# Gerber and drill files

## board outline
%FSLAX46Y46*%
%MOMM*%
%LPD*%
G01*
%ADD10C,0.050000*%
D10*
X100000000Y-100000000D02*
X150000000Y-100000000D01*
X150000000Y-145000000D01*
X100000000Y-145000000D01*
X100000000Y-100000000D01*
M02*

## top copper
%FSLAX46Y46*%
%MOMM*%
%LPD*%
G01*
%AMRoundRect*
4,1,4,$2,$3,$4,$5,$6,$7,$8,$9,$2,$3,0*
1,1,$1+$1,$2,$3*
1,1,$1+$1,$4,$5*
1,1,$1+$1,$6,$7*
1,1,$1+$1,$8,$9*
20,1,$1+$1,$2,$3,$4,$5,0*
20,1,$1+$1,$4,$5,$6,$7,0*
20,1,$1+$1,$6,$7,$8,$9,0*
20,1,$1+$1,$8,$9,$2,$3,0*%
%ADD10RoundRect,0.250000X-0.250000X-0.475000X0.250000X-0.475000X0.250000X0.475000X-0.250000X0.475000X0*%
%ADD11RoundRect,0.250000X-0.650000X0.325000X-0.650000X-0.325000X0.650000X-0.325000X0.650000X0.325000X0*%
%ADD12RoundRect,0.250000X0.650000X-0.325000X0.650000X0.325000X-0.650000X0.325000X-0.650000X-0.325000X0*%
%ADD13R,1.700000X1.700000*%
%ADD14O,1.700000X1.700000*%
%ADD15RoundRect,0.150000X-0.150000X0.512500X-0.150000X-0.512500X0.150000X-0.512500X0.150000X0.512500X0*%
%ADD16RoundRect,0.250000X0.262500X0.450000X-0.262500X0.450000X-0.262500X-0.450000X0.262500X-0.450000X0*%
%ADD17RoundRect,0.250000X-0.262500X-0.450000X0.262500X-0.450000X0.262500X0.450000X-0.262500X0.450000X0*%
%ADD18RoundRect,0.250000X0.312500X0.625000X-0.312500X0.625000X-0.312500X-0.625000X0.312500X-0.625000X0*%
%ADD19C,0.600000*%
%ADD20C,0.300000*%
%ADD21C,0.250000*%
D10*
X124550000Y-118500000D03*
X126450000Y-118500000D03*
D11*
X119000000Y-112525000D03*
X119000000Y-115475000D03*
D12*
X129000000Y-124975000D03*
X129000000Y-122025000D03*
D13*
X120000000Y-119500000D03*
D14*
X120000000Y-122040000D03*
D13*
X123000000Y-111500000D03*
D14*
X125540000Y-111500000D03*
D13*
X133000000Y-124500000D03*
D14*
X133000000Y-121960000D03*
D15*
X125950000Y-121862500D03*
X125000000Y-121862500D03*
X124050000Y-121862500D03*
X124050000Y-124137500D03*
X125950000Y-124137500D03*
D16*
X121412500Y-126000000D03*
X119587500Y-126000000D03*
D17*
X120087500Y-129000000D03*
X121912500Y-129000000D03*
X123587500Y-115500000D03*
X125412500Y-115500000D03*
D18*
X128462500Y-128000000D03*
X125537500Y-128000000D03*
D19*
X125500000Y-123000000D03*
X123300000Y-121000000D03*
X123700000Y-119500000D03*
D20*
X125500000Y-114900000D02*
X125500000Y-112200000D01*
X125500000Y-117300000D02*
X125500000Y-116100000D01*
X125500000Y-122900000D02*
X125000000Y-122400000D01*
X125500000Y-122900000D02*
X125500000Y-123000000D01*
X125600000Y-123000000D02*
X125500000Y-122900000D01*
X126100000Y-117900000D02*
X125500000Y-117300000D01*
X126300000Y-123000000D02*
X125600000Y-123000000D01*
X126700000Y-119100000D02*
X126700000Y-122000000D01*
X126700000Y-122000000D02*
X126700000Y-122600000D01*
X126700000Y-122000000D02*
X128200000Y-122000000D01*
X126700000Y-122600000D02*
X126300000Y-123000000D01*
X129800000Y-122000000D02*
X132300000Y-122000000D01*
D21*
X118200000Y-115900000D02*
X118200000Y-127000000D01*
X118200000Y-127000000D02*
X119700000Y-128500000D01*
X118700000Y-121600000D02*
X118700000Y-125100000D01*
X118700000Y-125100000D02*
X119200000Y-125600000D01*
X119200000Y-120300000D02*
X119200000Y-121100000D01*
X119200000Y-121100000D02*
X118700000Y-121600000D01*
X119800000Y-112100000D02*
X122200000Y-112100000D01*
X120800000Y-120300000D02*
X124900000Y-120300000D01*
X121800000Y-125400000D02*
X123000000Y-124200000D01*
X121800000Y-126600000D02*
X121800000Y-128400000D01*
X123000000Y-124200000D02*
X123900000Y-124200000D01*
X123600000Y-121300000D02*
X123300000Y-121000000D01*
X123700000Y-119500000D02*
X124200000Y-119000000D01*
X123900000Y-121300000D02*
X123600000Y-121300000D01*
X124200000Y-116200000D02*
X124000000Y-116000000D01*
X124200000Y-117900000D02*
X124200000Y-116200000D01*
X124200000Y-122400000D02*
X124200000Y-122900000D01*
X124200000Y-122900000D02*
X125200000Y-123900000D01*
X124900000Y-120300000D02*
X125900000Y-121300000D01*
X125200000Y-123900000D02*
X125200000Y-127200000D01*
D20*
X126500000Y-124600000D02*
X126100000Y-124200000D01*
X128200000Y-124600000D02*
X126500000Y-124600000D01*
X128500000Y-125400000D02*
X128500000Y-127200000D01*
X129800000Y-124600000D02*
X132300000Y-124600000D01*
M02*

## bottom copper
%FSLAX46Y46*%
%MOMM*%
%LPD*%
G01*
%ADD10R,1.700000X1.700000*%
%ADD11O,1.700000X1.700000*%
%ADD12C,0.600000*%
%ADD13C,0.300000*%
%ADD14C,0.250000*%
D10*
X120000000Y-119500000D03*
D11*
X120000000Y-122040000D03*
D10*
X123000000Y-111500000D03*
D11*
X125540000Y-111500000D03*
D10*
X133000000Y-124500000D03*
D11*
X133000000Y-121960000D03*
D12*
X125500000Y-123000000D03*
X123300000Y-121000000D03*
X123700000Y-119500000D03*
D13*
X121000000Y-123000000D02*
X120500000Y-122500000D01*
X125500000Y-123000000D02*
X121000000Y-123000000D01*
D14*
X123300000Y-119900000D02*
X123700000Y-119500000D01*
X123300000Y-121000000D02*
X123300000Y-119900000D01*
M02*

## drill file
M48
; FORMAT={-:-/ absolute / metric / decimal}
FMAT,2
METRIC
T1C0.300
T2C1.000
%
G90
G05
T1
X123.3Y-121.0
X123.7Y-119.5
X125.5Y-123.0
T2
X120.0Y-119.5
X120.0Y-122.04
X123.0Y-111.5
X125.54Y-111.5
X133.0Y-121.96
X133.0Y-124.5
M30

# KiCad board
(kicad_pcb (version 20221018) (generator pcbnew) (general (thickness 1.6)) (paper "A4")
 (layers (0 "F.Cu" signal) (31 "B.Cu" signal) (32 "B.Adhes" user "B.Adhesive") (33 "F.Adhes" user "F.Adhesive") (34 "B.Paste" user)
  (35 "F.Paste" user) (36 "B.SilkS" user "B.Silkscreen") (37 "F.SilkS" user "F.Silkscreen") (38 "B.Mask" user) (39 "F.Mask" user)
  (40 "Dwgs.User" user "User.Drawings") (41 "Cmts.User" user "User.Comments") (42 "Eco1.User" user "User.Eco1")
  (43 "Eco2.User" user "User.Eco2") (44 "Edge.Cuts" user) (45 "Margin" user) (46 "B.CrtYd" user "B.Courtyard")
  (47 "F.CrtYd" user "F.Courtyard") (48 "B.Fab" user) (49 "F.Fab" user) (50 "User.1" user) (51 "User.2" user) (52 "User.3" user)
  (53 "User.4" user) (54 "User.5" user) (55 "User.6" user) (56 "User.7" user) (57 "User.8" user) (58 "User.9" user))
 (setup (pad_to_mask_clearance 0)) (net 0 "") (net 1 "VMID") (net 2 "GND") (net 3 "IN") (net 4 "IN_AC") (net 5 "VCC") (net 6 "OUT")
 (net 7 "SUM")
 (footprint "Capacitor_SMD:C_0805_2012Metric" (layer "F.Cu") (at 125.5 118.5)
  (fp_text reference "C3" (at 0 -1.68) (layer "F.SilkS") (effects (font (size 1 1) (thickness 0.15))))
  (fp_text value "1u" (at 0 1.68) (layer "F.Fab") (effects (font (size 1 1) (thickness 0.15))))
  (pad "1" smd roundrect (at -0.95 0) (size 1 1.45) (layers "F.Cu" "F.Paste" "F.Mask") (roundrect_rratio 0.25) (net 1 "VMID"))
  (pad "2" smd roundrect (at 0.95 0) (size 1 1.45) (layers "F.Cu" "F.Paste" "F.Mask") (roundrect_rratio 0.25) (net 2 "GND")))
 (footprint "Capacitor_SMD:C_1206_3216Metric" (layer "F.Cu") (at 119 114 -90)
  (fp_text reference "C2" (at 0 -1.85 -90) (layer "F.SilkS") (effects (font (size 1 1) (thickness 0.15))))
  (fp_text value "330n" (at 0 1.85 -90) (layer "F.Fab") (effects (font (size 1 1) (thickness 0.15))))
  (pad "1" smd roundrect (at -1.475 0 270) (size 1.15 1.8) (layers "F.Cu" "F.Paste" "F.Mask") (roundrect_rratio 0.217391) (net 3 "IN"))
  (pad "2" smd roundrect (at 1.475 0 270) (size 1.15 1.8) (layers "F.Cu" "F.Paste" "F.Mask") (roundrect_rratio 0.217391) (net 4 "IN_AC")))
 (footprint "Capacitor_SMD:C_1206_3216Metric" (layer "F.Cu") (at 129 123.5 90)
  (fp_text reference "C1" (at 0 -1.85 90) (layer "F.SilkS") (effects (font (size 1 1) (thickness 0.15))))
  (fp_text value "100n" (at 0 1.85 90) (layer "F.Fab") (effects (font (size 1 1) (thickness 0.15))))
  (pad "1" smd roundrect (at -1.475 0 90) (size 1.15 1.8) (layers "F.Cu" "F.Paste" "F.Mask") (roundrect_rratio 0.217391) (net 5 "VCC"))
  (pad "2" smd roundrect (at 1.475 0 90) (size 1.15 1.8) (layers "F.Cu" "F.Paste" "F.Mask") (roundrect_rratio 0.217391) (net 2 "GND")))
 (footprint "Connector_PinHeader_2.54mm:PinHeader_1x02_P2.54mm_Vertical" (layer "F.Cu") (at 120 119.5)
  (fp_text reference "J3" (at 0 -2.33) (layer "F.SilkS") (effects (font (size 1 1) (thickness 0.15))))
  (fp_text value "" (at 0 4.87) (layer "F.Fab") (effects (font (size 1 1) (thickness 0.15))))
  (pad "1" thru_hole rect (at 0 0) (size 1.7 1.7) (drill 1) (layers "*.Cu" "*.Mask") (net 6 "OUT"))
  (pad "2" thru_hole oval (at 0 2.54) (size 1.7 1.7) (drill 1) (layers "*.Cu" "*.Mask") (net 2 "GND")))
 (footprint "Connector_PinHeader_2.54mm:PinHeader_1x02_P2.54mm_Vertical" (layer "F.Cu") (at 123 111.5 90)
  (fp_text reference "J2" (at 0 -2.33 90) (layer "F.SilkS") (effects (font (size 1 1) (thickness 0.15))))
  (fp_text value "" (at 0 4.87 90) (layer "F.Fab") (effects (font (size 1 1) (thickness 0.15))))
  (pad "1" thru_hole rect (at 0 0 90) (size 1.7 1.7) (drill 1) (layers "*.Cu" "*.Mask") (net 3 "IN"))
  (pad "2" thru_hole oval (at 0 2.54 90) (size 1.7 1.7) (drill 1) (layers "*.Cu" "*.Mask") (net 2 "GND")))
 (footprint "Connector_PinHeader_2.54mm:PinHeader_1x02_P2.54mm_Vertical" (layer "F.Cu") (at 133 124.5 180)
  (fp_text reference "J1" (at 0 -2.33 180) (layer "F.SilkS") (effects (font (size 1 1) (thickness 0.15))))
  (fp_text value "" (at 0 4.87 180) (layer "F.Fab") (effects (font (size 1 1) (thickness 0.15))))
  (pad "1" thru_hole rect (at 0 0 180) (size 1.7 1.7) (drill 1) (layers "*.Cu" "*.Mask") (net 5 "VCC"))
  (pad "2" thru_hole oval (at 0 2.54 180) (size 1.7 1.7) (drill 1) (layers "*.Cu" "*.Mask") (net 2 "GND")))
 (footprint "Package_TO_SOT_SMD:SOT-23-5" (layer "F.Cu") (at 125 123 -90)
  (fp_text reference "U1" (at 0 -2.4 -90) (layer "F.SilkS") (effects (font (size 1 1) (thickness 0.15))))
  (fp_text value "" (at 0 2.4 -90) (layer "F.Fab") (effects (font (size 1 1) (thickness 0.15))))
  (pad "1" smd roundrect (at -1.1375 -0.95 270) (size 1.325 0.6) (layers "F.Cu" "F.Paste" "F.Mask") (roundrect_rratio 0.25) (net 6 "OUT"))
  (pad "2" smd roundrect (at -1.1375 0 270) (size 1.325 0.6) (layers "F.Cu" "F.Paste" "F.Mask") (roundrect_rratio 0.25) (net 2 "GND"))
  (pad "3" smd roundrect (at -1.1375 0.95 270) (size 1.325 0.6) (layers "F.Cu" "F.Paste" "F.Mask") (roundrect_rratio 0.25) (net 1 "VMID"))
  (pad "4" smd roundrect (at 1.1375 0.95 270) (size 1.325 0.6) (layers "F.Cu" "F.Paste" "F.Mask") (roundrect_rratio 0.25) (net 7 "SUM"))
  (pad "5" smd roundrect (at 1.1375 -0.95 270) (size 1.325 0.6) (layers "F.Cu" "F.Paste" "F.Mask") (roundrect_rratio 0.25) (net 5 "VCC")))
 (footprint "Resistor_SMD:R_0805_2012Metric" (layer "F.Cu") (at 120.5 126 180)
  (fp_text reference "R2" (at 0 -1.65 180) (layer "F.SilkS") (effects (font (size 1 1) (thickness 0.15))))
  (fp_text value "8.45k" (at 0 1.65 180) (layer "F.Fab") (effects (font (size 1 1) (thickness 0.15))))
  (pad "1" smd roundrect (at -0.9125 0 180) (size 1.025 1.4) (layers "F.Cu" "F.Paste" "F.Mask") (roundrect_rratio 0.243902) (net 7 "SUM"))
  (pad "2" smd roundrect (at 0.9125 0 180) (size 1.025 1.4) (layers "F.Cu" "F.Paste" "F.Mask") (roundrect_rratio 0.243902) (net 6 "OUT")))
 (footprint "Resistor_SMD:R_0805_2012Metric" (layer "F.Cu") (at 121 129)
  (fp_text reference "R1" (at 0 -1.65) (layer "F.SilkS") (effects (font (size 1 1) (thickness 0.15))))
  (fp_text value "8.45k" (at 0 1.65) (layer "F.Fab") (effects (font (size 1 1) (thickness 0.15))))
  (pad "1" smd roundrect (at -0.9125 0) (size 1.025 1.4) (layers "F.Cu" "F.Paste" "F.Mask") (roundrect_rratio 0.243902) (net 4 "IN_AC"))
  (pad "2" smd roundrect (at 0.9125 0) (size 1.025 1.4) (layers "F.Cu" "F.Paste" "F.Mask") (roundrect_rratio 0.243902) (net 7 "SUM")))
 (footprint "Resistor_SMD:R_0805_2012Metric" (layer "F.Cu") (at 124.5 115.5)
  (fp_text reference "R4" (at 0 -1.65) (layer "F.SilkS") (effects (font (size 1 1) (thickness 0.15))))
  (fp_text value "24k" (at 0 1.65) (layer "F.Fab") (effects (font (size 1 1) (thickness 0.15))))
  (pad "1" smd roundrect (at -0.9125 0) (size 1.025 1.4) (layers "F.Cu" "F.Paste" "F.Mask") (roundrect_rratio 0.243902) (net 1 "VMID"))
  (pad "2" smd roundrect (at 0.9125 0) (size 1.025 1.4) (layers "F.Cu" "F.Paste" "F.Mask") (roundrect_rratio 0.243902) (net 2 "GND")))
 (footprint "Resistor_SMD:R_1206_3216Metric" (layer "F.Cu") (at 127 128 180)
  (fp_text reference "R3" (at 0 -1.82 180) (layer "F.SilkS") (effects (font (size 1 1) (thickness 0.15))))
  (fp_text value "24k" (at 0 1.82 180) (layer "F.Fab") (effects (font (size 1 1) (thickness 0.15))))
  (pad "1" smd roundrect (at -1.4625 0 180) (size 1.125 1.75) (layers "F.Cu" "F.Paste" "F.Mask") (roundrect_rratio 0.222222) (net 5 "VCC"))
  (pad "2" smd roundrect (at 1.4625 0 180) (size 1.125 1.75) (layers "F.Cu" "F.Paste" "F.Mask") (roundrect_rratio 0.222222) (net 1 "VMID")))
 (gr_rect (start 100 100) (end 150 145) (stroke (width 0.05) (type default)) (fill none) (layer "Edge.Cuts"))
 (segment (start 125.5 114.9) (end 125.5 112.2) (width 0.3) (layer "F.Cu") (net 2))
 (segment (start 125.5 117.3) (end 125.5 116.1) (width 0.3) (layer "F.Cu") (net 2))
 (segment (start 125.5 122.9) (end 125 122.4) (width 0.3) (layer "F.Cu") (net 2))
 (segment (start 125.5 122.9) (end 125.5 123) (width 0.3) (layer "F.Cu") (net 2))
 (segment (start 125.6 123) (end 125.5 122.9) (width 0.3) (layer "F.Cu") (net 2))
 (segment (start 126.1 117.9) (end 125.5 117.3) (width 0.3) (layer "F.Cu") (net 2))
 (segment (start 126.3 123) (end 125.6 123) (width 0.3) (layer "F.Cu") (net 2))
 (segment (start 126.7 119.1) (end 126.7 122) (width 0.3) (layer "F.Cu") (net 2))
 (segment (start 126.7 122) (end 126.7 122.6) (width 0.3) (layer "F.Cu") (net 2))
 (segment (start 126.7 122) (end 128.2 122) (width 0.3) (layer "F.Cu") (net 2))
 (segment (start 126.7 122.6) (end 126.3 123) (width 0.3) (layer "F.Cu") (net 2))
 (segment (start 129.8 122) (end 132.3 122) (width 0.3) (layer "F.Cu") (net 2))
 (via (at 125.5 123) (size 0.6) (drill 0.3) (layers "F.Cu" "B.Cu") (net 2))
 (segment (start 118.2 115.9) (end 118.2 127) (width 0.25) (layer "F.Cu") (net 4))
 (segment (start 118.2 127) (end 119.7 128.5) (width 0.25) (layer "F.Cu") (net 4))
 (segment (start 118.7 121.6) (end 118.7 125.1) (width 0.25) (layer "F.Cu") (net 6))
 (segment (start 118.7 125.1) (end 119.2 125.6) (width 0.25) (layer "F.Cu") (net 6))
 (segment (start 119.2 120.3) (end 119.2 121.1) (width 0.25) (layer "F.Cu") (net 6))
 (segment (start 119.2 121.1) (end 118.7 121.6) (width 0.25) (layer "F.Cu") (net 6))
 (segment (start 119.8 112.1) (end 122.2 112.1) (width 0.25) (layer "F.Cu") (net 3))
 (segment (start 120.8 120.3) (end 124.9 120.3) (width 0.25) (layer "F.Cu") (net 6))
 (segment (start 121 123) (end 120.5 122.5) (width 0.3) (layer "B.Cu") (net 2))
 (segment (start 121.8 125.4) (end 123 124.2) (width 0.25) (layer "F.Cu") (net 7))
 (segment (start 121.8 126.6) (end 121.8 128.4) (width 0.25) (layer "F.Cu") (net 7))
 (segment (start 123 124.2) (end 123.9 124.2) (width 0.25) (layer "F.Cu") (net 7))
 (segment (start 123.6 121.3) (end 123.3 121) (width 0.25) (layer "F.Cu") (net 1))
 (segment (start 123.7 119.5) (end 124.2 119) (width 0.25) (layer "F.Cu") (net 1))
 (segment (start 123.9 121.3) (end 123.6 121.3) (width 0.25) (layer "F.Cu") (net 1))
 (segment (start 124.2 116.2) (end 124 116) (width 0.25) (layer "F.Cu") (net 1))
 (segment (start 124.2 117.9) (end 124.2 116.2) (width 0.25) (layer "F.Cu") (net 1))
 (segment (start 124.2 122.4) (end 124.2 122.9) (width 0.25) (layer "F.Cu") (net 1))
 (segment (start 124.2 122.9) (end 125.2 123.9) (width 0.25) (layer "F.Cu") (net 1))
 (segment (start 124.9 120.3) (end 125.9 121.3) (width 0.25) (layer "F.Cu") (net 6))
 (segment (start 125.2 123.9) (end 125.2 127.2) (width 0.25) (layer "F.Cu") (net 1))
 (segment (start 125.5 123) (end 121 123) (width 0.3) (layer "B.Cu") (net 2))
 (segment (start 126.5 124.6) (end 126.1 124.2) (width 0.3) (layer "F.Cu") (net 5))
 (segment (start 128.2 124.6) (end 126.5 124.6) (width 0.3) (layer "F.Cu") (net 5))
 (segment (start 128.5 125.4) (end 128.5 127.2) (width 0.3) (layer "F.Cu") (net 5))
 (segment (start 129.8 124.6) (end 132.3 124.6) (width 0.3) (layer "F.Cu") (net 5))
 (via (at 123.3 121) (size 0.6) (drill 0.3) (layers "F.Cu" "B.Cu") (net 1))
 (via (at 123.7 119.5) (size 0.6) (drill 0.3) (layers "F.Cu" "B.Cu") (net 1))
 (segment (start 123.3 119.9) (end 123.7 119.5) (width 0.25) (layer "B.Cu") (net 1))
 (segment (start 123.3 121) (end 123.3 119.9) (width 0.25) (layer "B.Cu") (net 1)))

